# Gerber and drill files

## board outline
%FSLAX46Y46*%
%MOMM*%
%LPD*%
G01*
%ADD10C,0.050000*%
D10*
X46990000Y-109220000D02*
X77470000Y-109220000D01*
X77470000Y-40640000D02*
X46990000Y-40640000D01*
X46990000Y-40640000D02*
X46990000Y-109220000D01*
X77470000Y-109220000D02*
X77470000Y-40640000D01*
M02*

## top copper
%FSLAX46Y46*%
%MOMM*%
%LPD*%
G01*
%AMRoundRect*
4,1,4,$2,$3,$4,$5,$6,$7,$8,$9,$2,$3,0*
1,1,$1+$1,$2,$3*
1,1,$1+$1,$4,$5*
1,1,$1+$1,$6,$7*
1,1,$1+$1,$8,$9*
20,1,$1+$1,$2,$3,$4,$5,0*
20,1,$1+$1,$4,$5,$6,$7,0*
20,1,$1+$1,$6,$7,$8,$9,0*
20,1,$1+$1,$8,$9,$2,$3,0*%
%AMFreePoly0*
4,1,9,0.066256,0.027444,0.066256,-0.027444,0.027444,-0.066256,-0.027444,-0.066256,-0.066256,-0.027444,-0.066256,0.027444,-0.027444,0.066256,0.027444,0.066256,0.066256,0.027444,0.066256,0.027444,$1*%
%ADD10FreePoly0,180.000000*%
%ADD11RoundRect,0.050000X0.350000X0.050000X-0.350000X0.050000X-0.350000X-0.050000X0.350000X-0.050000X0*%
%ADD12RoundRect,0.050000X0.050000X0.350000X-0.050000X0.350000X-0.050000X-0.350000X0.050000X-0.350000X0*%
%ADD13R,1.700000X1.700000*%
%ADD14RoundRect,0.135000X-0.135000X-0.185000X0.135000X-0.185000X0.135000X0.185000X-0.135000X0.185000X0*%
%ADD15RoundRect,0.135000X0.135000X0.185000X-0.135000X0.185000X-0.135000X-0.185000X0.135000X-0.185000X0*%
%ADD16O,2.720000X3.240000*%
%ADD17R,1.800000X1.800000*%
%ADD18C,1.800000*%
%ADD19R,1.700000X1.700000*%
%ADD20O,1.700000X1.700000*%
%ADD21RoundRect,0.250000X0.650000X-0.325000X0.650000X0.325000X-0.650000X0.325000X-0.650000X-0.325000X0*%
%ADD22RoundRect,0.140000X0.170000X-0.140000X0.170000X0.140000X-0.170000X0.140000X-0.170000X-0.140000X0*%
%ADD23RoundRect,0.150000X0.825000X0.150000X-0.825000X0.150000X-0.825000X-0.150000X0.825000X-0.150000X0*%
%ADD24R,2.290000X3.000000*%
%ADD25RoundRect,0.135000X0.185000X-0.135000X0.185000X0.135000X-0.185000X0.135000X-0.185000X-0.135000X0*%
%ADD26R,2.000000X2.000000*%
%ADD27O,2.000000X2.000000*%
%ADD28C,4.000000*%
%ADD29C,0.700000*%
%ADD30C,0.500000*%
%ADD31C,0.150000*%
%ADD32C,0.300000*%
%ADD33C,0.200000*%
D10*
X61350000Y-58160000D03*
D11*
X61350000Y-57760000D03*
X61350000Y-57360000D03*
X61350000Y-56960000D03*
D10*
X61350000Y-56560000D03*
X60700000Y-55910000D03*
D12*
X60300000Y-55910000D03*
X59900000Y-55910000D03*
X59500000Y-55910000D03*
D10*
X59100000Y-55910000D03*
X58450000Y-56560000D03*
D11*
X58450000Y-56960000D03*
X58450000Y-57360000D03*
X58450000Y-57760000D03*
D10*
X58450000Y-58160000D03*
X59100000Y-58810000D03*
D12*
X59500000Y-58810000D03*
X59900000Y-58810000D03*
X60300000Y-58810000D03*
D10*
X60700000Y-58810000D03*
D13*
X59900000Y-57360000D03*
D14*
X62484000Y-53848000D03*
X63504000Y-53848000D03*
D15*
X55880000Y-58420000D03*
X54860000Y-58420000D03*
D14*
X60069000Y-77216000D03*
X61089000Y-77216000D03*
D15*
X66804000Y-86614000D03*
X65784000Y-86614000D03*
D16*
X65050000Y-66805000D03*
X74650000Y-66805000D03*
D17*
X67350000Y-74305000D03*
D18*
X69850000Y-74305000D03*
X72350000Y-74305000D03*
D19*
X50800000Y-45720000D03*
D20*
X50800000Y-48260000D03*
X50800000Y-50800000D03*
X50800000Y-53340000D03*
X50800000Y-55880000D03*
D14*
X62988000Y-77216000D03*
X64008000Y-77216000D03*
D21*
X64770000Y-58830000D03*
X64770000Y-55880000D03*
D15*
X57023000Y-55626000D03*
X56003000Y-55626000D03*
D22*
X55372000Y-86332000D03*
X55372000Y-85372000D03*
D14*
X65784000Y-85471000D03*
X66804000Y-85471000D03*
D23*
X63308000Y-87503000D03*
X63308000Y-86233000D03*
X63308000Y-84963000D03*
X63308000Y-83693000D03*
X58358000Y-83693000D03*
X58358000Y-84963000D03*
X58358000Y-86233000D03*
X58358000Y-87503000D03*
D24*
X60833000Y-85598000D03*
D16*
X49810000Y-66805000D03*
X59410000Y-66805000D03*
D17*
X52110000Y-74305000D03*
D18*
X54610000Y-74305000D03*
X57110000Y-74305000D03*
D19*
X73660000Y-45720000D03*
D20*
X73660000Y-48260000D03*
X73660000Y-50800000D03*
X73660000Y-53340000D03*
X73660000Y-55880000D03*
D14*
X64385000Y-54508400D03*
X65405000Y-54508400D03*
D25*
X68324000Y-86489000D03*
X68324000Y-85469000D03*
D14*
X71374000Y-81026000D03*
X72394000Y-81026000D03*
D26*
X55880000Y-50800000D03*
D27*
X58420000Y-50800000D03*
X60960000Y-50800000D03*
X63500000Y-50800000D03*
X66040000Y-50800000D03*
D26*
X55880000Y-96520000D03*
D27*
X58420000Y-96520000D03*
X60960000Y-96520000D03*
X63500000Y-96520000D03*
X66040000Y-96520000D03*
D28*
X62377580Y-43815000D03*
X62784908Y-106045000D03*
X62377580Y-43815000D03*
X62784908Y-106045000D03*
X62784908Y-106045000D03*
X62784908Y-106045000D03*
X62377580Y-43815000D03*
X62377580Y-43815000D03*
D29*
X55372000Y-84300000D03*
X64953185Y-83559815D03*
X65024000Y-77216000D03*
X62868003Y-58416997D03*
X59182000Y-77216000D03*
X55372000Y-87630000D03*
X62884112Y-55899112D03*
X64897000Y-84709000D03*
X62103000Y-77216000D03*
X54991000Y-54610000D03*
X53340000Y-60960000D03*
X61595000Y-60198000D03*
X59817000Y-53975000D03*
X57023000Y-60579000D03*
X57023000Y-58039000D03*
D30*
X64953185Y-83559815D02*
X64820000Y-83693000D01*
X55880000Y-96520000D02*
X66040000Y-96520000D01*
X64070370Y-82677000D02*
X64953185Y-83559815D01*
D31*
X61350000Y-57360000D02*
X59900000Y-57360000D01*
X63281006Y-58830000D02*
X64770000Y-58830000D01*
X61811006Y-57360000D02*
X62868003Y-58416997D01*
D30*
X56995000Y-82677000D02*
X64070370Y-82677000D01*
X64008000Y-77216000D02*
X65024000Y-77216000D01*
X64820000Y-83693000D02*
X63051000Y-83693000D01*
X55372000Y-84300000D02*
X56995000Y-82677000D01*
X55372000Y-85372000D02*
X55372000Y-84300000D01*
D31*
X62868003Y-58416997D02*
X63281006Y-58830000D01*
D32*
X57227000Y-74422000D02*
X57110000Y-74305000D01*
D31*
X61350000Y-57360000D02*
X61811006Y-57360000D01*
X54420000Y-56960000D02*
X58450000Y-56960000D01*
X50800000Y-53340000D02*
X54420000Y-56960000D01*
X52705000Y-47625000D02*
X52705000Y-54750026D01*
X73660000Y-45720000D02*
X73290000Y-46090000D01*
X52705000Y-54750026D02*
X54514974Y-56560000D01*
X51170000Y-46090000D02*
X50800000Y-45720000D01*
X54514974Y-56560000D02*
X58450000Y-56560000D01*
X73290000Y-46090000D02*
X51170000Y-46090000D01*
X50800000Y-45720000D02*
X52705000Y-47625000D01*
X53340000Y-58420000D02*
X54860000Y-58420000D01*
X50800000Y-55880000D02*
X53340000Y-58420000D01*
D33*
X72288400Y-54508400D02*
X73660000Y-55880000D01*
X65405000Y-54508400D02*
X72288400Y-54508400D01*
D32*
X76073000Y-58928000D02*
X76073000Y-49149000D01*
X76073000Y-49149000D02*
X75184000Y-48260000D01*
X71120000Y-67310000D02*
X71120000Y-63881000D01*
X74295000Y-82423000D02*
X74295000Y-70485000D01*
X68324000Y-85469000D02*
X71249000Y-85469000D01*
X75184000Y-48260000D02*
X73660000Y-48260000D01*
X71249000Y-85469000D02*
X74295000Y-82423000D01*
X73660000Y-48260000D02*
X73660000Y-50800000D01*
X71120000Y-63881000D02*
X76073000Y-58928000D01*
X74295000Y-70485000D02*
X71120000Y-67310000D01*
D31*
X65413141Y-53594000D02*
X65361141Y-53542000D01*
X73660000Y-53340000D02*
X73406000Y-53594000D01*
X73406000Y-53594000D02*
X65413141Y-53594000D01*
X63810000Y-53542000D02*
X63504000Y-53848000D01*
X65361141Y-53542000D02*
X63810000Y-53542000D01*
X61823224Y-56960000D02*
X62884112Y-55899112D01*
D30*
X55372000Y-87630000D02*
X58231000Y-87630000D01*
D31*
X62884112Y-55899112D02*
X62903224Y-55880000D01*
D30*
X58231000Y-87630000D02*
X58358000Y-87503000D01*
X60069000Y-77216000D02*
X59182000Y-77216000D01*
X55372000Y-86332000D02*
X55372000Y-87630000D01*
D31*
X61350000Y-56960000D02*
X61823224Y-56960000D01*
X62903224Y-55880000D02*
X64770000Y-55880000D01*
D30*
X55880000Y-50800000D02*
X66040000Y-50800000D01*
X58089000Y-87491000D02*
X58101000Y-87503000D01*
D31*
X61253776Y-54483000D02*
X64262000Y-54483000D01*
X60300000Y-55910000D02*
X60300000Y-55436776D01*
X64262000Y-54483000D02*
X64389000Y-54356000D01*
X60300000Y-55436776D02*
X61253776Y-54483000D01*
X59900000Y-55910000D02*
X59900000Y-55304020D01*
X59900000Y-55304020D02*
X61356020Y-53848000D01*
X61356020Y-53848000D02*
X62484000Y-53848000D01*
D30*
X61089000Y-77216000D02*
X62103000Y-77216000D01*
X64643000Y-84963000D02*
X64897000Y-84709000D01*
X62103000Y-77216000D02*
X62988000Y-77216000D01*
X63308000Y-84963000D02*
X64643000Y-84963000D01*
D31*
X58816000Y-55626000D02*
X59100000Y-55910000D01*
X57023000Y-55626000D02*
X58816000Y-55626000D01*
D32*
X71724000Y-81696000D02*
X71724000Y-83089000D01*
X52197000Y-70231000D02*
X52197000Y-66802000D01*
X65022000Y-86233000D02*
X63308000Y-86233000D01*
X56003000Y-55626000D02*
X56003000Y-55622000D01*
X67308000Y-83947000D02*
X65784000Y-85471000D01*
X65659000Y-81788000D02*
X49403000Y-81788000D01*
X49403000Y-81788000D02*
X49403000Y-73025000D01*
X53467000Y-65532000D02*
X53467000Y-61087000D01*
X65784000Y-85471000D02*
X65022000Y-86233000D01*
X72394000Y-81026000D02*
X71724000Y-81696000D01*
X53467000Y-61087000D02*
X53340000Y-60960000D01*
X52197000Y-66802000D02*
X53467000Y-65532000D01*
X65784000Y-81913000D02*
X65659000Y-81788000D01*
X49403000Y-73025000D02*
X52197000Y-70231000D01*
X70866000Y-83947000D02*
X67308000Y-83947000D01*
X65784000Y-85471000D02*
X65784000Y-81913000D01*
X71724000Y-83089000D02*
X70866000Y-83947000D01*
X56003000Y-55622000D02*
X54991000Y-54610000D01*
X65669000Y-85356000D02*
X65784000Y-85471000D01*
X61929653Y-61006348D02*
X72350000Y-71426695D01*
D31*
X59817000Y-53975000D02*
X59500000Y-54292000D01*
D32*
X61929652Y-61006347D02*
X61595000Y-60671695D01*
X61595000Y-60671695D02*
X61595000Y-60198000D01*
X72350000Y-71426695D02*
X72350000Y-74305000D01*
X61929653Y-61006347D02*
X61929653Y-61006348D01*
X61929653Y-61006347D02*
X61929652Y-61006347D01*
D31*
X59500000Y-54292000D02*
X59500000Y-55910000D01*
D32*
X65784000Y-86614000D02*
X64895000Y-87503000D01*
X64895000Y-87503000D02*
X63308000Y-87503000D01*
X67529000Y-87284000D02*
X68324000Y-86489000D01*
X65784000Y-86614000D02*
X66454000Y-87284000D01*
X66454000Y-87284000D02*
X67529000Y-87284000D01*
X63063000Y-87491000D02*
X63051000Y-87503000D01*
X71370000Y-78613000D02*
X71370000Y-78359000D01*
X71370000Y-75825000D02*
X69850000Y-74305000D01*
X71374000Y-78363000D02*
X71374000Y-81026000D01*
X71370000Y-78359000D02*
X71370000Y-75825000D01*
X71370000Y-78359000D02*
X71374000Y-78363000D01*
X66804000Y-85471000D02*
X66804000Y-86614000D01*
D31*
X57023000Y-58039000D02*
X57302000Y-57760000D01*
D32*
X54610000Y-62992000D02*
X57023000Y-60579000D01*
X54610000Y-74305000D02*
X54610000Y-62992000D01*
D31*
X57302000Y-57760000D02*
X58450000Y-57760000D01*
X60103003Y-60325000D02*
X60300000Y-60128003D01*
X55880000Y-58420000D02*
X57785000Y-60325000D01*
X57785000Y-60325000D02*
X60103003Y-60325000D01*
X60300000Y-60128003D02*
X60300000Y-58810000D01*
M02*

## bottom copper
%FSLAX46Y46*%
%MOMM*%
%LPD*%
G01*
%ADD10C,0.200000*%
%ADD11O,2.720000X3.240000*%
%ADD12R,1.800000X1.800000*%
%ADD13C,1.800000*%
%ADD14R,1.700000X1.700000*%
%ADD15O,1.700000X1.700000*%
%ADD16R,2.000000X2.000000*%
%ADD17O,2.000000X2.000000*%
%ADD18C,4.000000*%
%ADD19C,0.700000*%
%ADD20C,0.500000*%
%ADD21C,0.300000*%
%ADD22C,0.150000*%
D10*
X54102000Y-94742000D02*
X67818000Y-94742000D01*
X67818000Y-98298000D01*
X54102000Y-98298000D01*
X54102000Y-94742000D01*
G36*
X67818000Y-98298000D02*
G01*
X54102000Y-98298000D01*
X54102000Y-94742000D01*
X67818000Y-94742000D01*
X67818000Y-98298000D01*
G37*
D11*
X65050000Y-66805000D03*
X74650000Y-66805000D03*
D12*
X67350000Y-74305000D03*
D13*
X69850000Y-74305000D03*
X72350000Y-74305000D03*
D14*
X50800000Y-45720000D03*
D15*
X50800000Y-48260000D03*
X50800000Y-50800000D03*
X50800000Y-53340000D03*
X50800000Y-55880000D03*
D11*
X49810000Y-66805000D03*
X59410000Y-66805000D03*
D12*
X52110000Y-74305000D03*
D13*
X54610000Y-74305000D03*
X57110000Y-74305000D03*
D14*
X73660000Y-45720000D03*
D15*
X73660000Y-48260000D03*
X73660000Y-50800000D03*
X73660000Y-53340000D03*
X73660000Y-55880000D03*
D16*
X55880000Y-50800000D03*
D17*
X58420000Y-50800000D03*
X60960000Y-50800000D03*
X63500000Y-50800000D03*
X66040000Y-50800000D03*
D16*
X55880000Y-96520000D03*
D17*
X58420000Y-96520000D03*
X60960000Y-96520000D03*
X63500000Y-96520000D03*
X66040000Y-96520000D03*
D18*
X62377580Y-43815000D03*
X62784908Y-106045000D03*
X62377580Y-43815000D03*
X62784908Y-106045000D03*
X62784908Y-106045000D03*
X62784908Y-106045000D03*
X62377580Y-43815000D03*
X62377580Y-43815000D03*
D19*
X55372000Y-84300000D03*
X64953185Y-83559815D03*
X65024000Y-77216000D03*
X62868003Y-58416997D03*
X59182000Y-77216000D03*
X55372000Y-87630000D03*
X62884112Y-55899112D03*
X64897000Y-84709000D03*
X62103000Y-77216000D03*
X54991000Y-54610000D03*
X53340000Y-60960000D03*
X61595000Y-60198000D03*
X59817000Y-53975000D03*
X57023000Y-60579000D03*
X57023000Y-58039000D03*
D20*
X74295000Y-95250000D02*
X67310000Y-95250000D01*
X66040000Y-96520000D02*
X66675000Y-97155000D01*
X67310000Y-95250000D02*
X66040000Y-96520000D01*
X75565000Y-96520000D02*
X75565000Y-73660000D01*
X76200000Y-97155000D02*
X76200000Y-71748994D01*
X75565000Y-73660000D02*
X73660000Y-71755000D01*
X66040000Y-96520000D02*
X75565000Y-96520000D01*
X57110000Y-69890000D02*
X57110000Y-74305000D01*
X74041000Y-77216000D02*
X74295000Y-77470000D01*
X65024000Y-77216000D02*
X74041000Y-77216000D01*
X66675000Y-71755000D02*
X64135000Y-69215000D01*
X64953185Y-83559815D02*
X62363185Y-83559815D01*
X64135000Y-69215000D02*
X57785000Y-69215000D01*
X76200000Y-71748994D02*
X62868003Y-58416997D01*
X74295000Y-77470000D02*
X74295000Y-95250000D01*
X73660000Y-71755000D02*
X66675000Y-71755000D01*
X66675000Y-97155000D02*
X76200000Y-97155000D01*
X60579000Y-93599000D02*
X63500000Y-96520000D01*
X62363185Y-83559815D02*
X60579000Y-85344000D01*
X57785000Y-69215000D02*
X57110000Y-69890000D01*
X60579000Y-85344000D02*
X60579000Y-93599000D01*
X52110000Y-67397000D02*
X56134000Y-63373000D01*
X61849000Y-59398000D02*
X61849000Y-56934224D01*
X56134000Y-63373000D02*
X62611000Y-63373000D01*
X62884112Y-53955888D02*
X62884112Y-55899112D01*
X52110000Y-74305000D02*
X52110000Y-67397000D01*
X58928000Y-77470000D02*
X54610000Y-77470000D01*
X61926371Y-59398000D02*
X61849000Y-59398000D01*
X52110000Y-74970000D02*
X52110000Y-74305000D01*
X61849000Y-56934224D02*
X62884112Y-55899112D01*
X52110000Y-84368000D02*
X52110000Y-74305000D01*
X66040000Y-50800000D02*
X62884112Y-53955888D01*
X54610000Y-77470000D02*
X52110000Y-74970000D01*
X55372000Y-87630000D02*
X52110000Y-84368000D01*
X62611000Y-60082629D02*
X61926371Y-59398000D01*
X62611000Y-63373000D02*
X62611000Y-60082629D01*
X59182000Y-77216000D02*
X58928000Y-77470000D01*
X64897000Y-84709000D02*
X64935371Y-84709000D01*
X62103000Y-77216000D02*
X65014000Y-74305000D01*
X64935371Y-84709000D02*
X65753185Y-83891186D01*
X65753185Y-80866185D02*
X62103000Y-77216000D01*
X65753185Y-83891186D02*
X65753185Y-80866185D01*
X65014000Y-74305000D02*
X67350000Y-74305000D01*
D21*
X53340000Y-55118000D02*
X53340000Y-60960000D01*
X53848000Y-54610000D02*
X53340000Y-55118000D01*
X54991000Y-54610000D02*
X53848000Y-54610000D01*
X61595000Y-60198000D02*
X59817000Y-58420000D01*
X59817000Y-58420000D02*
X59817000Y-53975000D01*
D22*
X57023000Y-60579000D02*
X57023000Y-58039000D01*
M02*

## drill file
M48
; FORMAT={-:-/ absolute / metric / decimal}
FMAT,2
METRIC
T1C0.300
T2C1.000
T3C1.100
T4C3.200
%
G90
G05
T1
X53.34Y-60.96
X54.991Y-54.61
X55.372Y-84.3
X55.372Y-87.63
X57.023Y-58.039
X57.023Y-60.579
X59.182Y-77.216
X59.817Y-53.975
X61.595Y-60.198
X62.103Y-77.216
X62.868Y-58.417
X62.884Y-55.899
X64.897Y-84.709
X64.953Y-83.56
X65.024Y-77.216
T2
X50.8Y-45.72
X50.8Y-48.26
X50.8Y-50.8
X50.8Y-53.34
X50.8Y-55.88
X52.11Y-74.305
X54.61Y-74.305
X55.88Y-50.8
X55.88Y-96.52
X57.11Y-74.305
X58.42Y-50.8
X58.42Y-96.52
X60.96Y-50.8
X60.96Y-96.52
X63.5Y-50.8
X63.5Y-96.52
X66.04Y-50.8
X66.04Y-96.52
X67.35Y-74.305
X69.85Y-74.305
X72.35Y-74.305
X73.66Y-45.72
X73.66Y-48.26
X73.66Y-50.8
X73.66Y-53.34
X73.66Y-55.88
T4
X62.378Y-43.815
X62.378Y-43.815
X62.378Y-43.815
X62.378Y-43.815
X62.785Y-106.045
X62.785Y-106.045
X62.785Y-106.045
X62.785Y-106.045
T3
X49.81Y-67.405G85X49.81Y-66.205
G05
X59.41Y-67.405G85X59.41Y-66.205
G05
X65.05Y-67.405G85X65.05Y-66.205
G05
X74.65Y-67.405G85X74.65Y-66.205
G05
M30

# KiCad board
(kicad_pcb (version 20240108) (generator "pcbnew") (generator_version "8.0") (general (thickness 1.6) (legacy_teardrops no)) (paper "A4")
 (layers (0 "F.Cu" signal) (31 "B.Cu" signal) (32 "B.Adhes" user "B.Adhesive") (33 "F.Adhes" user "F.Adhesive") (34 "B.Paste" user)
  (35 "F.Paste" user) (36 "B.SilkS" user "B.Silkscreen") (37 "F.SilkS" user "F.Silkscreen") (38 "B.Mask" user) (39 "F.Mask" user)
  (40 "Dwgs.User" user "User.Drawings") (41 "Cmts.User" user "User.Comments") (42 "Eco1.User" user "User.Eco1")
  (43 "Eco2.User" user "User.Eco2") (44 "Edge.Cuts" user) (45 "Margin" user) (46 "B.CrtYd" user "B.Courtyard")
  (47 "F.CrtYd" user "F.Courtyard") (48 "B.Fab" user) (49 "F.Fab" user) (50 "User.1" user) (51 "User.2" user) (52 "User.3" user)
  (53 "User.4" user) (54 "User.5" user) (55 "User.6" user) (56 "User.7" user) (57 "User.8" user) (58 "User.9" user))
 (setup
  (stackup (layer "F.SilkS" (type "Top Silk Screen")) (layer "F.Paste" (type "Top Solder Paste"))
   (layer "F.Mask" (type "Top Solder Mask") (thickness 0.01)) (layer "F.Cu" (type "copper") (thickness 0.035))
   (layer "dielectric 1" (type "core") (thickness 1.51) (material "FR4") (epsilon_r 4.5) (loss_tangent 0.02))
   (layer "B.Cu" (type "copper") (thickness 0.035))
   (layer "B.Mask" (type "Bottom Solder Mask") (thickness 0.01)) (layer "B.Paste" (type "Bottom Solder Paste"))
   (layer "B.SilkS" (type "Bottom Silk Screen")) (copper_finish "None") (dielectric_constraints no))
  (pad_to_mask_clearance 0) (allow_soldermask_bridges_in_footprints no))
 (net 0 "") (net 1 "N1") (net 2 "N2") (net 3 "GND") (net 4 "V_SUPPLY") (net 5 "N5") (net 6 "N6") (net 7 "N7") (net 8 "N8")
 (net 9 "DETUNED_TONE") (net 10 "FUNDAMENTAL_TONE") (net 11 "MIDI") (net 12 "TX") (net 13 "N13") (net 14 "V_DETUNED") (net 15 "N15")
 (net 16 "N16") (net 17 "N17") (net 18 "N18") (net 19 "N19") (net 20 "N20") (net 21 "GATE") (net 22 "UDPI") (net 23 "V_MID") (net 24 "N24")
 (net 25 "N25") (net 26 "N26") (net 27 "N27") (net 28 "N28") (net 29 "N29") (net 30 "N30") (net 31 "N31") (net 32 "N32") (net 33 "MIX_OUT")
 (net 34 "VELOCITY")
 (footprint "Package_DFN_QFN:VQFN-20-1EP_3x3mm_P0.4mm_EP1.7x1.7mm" (layer "F.Cu") (at 59.9 57.36 180)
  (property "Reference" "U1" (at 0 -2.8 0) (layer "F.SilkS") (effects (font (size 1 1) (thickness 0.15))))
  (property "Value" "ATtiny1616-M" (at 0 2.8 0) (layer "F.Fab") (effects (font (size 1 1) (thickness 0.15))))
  (pad "" smd roundrect (at -0.425 -0.425 180) (size 0.69 0.69) (layers "F.Paste") (roundrect_rratio 0.25))
  (pad "" smd roundrect (at -0.425 0.425 180) (size 0.69 0.69) (layers "F.Paste") (roundrect_rratio 0.25))
  (pad "" smd roundrect (at 0.425 -0.425 180) (size 0.69 0.69) (layers "F.Paste") (roundrect_rratio 0.25))
  (pad "" smd roundrect (at 0.425 0.425 180) (size 0.69 0.69) (layers "F.Paste") (roundrect_rratio 0.25))
  (pad "1" smd custom (at -1.45 -0.8 180) (size 0.143431 0.143431) (layers "F.Cu" "F.Paste" "F.Mask") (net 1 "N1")
   (options (clearance outline) (anchor circle)) (primitives))
  (pad "2" smd roundrect (at -1.45 -0.4 180) (size 0.8 0.2) (layers "F.Cu" "F.Paste" "F.Mask") (roundrect_rratio 0.25) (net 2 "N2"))
  (pad "3" smd roundrect (at -1.45 0 180) (size 0.8 0.2) (layers "F.Cu" "F.Paste" "F.Mask") (roundrect_rratio 0.25) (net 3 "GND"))
  (pad "4" smd roundrect (at -1.45 0.4 180) (size 0.8 0.2) (layers "F.Cu" "F.Paste" "F.Mask") (roundrect_rratio 0.25) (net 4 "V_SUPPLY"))
  (pad "5" smd custom (at -1.45 0.8 180) (size 0.143431 0.143431) (layers "F.Cu" "F.Paste" "F.Mask") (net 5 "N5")
   (options (clearance outline) (anchor circle)) (primitives))
  (pad "6" smd custom (at -0.8 1.45 180) (size 0.143431 0.143431) (layers "F.Cu" "F.Paste" "F.Mask") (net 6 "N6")
   (options (clearance outline) (anchor circle)) (primitives))
  (pad "7" smd roundrect (at -0.4 1.45 180) (size 0.2 0.8) (layers "F.Cu" "F.Paste" "F.Mask") (roundrect_rratio 0.25) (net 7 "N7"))
  (pad "8" smd roundrect (at 0 1.45 180) (size 0.2 0.8) (layers "F.Cu" "F.Paste" "F.Mask") (roundrect_rratio 0.25) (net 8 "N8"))
  (pad "9" smd roundrect (at 0.4 1.45 180) (size 0.2 0.8) (layers "F.Cu" "F.Paste" "F.Mask") (roundrect_rratio 0.25) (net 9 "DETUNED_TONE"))
  (pad "10" smd custom (at 0.8 1.45 180) (size 0.143431 0.143431) (layers "F.Cu" "F.Paste" "F.Mask") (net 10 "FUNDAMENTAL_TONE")
   (options (clearance outline) (anchor circle)) (primitives))
  (pad "11" smd custom (at 1.45 0.8 180) (size 0.143431 0.143431) (layers "F.Cu" "F.Paste" "F.Mask") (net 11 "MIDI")
   (options (clearance outline) (anchor circle)) (primitives))
  (pad "12" smd roundrect (at 1.45 0.4 180) (size 0.8 0.2) (layers "F.Cu" "F.Paste" "F.Mask") (roundrect_rratio 0.25) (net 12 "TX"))
  (pad "13" smd roundrect (at 1.45 0 180) (size 0.8 0.2) (layers "F.Cu" "F.Paste" "F.Mask") (roundrect_rratio 0.25) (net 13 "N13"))
  (pad "14" smd roundrect (at 1.45 -0.4 180) (size 0.8 0.2) (layers "F.Cu" "F.Paste" "F.Mask") (roundrect_rratio 0.25) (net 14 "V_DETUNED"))
  (pad "15" smd custom (at 1.45 -0.8 180) (size 0.143431 0.143431) (layers "F.Cu" "F.Paste" "F.Mask") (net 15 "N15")
   (options (clearance outline) (anchor circle)) (primitives))
  (pad "16" smd custom (at 0.8 -1.45 180) (size 0.143431 0.143431) (layers "F.Cu" "F.Paste" "F.Mask") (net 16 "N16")
   (options (clearance outline) (anchor circle)) (primitives))
  (pad "17" smd roundrect (at 0.4 -1.45 180) (size 0.2 0.8) (layers "F.Cu" "F.Paste" "F.Mask") (roundrect_rratio 0.25) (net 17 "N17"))
  (pad "18" smd roundrect (at 0 -1.45 180) (size 0.2 0.8) (layers "F.Cu" "F.Paste" "F.Mask") (roundrect_rratio 0.25) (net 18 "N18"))
  (pad "19" smd roundrect (at -0.4 -1.45 180) (size 0.2 0.8) (layers "F.Cu" "F.Paste" "F.Mask") (roundrect_rratio 0.25) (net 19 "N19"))
  (pad "20" smd custom (at -0.8 -1.45 180) (size 0.143431 0.143431) (layers "F.Cu" "F.Paste" "F.Mask") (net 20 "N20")
   (options (clearance outline) (anchor circle)) (primitives))
  (pad "21" smd rect (at 0 0 180) (size 1.7 1.7) (layers "F.Cu" "F.Mask") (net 3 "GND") (zone_connect 2)))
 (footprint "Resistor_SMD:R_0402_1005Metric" (layer "F.Cu") (at 62.994 53.848)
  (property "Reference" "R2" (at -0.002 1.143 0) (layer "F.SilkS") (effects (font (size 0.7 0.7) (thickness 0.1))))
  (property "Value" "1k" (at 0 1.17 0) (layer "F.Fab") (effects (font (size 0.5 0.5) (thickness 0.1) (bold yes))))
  (pad "1" smd roundrect (at -0.51 0) (size 0.54 0.64) (layers "F.Cu" "F.Paste" "F.Mask") (roundrect_rratio 0.25) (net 8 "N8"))
  (pad "2" smd roundrect (at 0.51 0) (size 0.54 0.64) (layers "F.Cu" "F.Paste" "F.Mask") (roundrect_rratio 0.25) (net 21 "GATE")))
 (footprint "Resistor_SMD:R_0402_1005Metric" (layer "F.Cu") (at 55.37 58.42 180)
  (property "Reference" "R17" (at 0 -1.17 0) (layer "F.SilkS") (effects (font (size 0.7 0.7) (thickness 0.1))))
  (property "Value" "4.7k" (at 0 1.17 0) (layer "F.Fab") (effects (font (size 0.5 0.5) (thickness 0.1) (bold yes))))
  (pad "1" smd roundrect (at -0.51 0 180) (size 0.54 0.64) (layers "F.Cu" "F.Paste" "F.Mask") (roundrect_rratio 0.25) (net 19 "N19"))
  (pad "2" smd roundrect (at 0.51 0 180) (size 0.54 0.64) (layers "F.Cu" "F.Paste" "F.Mask") (roundrect_rratio 0.25) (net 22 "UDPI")))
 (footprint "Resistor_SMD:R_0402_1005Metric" (layer "F.Cu") (at 60.579 77.216)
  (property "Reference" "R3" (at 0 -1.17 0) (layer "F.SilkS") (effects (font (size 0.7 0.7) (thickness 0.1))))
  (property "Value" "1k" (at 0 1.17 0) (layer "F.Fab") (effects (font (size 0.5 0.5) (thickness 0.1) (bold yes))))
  (pad "1" smd roundrect (at -0.51 0) (size 0.54 0.64) (layers "F.Cu" "F.Paste" "F.Mask") (roundrect_rratio 0.25) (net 4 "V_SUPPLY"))
  (pad "2" smd roundrect (at 0.51 0) (size 0.54 0.64) (layers "F.Cu" "F.Paste" "F.Mask") (roundrect_rratio 0.25) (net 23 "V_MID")))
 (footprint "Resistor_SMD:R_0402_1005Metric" (layer "F.Cu") (at 66.294 86.614 180)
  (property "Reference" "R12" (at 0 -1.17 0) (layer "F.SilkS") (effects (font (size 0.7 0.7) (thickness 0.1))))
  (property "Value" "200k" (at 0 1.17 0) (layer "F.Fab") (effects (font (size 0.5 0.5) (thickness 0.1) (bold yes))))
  (pad "1" smd roundrect (at -0.51 0 180) (size 0.54 0.64) (layers "F.Cu" "F.Paste" "F.Mask") (roundrect_rratio 0.25) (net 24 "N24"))
  (pad "2" smd roundrect (at 0.51 0 180) (size 0.54 0.64) (layers "F.Cu" "F.Paste" "F.Mask") (roundrect_rratio 0.25) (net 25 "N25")))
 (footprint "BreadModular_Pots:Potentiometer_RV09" (layer "F.Cu") (at 67.35 74.305 90)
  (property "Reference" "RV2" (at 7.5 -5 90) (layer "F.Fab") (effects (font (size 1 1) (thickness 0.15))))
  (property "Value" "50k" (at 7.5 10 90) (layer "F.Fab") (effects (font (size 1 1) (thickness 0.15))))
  (pad "" thru_hole oval (at 7.5 -2.3 180) (size 2.72 3.24) (drill oval 1.1 2.3) (layers "*.Cu" "*.Mask") (remove_unused_layers no))
  (pad "" thru_hole oval (at 7.5 7.3 180) (size 2.72 3.24) (drill oval 1.1 2.3) (layers "*.Cu" "*.Mask") (remove_unused_layers no))
  (pad "1" thru_hole rect (at 0 0 180) (size 1.8 1.8) (drill 1) (layers "*.Cu" "*.Mask") (remove_unused_layers no) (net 23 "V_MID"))
  (pad "2" thru_hole circle (at 0 2.5 180) (size 1.8 1.8) (drill 1) (layers "*.Cu" "*.Mask") (remove_unused_layers no) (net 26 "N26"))
  (pad "3" thru_hole circle (at 0 5 180) (size 1.8 1.8) (drill 1) (layers "*.Cu" "*.Mask") (remove_unused_layers no) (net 9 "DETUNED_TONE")))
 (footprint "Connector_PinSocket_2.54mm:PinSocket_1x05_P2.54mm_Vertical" (layer "F.Cu") (at 50.8 45.72)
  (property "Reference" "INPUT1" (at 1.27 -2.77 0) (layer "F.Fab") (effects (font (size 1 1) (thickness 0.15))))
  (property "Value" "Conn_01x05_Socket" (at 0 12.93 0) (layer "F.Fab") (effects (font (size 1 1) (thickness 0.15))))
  (pad "1" thru_hole rect (at 0 0) (size 1.7 1.7) (drill 1) (layers "*.Cu" "*.Mask") (remove_unused_layers no) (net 11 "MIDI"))
  (pad "2" thru_hole oval (at 0 2.54) (size 1.7 1.7) (drill 1) (layers "*.Cu" "*.Mask") (remove_unused_layers no) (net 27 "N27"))
  (pad "3" thru_hole oval (at 0 5.08) (size 1.7 1.7) (drill 1) (layers "*.Cu" "*.Mask") (remove_unused_layers no) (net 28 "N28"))
  (pad "4" thru_hole oval (at 0 7.62) (size 1.7 1.7) (drill 1) (layers "*.Cu" "*.Mask") (remove_unused_layers no) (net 12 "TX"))
  (pad "5" thru_hole oval (at 0 10.16) (size 1.7 1.7) (drill 1) (layers "*.Cu" "*.Mask") (remove_unused_layers no) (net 22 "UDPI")))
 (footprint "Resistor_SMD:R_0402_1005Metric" (layer "F.Cu") (at 63.498 77.216)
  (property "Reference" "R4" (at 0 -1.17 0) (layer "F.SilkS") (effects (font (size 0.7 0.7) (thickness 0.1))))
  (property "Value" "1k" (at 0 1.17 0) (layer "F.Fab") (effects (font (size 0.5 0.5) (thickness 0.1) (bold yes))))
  (pad "1" smd roundrect (at -0.51 0) (size 0.54 0.64) (layers "F.Cu" "F.Paste" "F.Mask") (roundrect_rratio 0.25) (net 23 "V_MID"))
  (pad "2" smd roundrect (at 0.51 0) (size 0.54 0.64) (layers "F.Cu" "F.Paste" "F.Mask") (roundrect_rratio 0.25) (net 3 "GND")))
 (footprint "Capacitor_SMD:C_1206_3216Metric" (layer "F.Cu") (at 64.77 57.355 90)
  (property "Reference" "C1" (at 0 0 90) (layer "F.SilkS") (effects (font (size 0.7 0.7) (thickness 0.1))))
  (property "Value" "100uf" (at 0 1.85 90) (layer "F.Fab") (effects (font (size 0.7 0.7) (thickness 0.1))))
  (pad "1" smd roundrect (at -1.475 0 90) (size 1.15 1.8) (layers "F.Cu" "F.Paste" "F.Mask") (roundrect_rratio 0.217391) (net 3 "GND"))
  (pad "2" smd roundrect (at 1.475 0 90) (size 1.15 1.8) (layers "F.Cu" "F.Paste" "F.Mask") (roundrect_rratio 0.217391) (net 4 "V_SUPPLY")))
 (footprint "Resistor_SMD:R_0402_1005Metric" (layer "F.Cu") (at 56.513 55.626 180)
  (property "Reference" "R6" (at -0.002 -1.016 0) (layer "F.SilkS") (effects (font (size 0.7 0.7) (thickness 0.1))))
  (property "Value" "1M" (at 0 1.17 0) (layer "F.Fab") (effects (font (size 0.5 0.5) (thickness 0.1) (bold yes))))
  (pad "1" smd roundrect (at -0.51 0 180) (size 0.54 0.64) (layers "F.Cu" "F.Paste" "F.Mask") (roundrect_rratio 0.25)
   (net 10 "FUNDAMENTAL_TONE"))
  (pad "2" smd roundrect (at 0.51 0 180) (size 0.54 0.64) (layers "F.Cu" "F.Paste" "F.Mask") (roundrect_rratio 0.25) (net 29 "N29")))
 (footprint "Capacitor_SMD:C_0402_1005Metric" (layer "F.Cu") (at 55.372 85.852 90)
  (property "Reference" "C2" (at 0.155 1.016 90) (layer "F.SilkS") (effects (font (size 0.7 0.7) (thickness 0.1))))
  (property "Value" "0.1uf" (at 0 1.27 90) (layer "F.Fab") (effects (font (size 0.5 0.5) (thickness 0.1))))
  (pad "1" smd roundrect (at -0.48 0 90) (size 0.56 0.62) (layers "F.Cu" "F.Paste" "F.Mask") (roundrect_rratio 0.25) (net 4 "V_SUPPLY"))
  (pad "2" smd roundrect (at 0.48 0 90) (size 0.56 0.62) (layers "F.Cu" "F.Paste" "F.Mask") (roundrect_rratio 0.25) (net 3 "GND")))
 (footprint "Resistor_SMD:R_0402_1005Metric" (layer "F.Cu") (at 66.294 85.471)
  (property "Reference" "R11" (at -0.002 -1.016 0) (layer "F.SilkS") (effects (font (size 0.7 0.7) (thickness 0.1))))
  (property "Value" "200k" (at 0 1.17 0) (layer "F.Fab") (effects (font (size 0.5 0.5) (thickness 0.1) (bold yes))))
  (pad "1" smd roundrect (at -0.51 0) (size 0.54 0.64) (layers "F.Cu" "F.Paste" "F.Mask") (roundrect_rratio 0.25) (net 29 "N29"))
  (pad "2" smd roundrect (at 0.51 0) (size 0.54 0.64) (layers "F.Cu" "F.Paste" "F.Mask") (roundrect_rratio 0.25) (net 24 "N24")))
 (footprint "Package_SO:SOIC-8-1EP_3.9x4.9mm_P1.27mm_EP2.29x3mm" (layer "F.Cu") (at 60.833 85.598 180)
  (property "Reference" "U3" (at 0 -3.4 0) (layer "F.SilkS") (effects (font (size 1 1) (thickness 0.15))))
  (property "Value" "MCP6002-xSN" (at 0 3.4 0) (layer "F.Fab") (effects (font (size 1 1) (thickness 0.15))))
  (pad "" smd roundrect (at -0.57 -0.75 180) (size 0.92 1.21) (layers "F.Paste") (roundrect_rratio 0.25))
  (pad "" smd roundrect (at -0.57 0.75 180) (size 0.92 1.21) (layers "F.Paste") (roundrect_rratio 0.25))
  (pad "" smd roundrect (at 0.57 -0.75 180) (size 0.92 1.21) (layers "F.Paste") (roundrect_rratio 0.25))
  (pad "" smd roundrect (at 0.57 0.75 180) (size 0.92 1.21) (layers "F.Paste") (roundrect_rratio 0.25))
  (pad "1" smd roundrect (at -2.475 -1.905 180) (size 1.95 0.6) (layers "F.Cu" "F.Paste" "F.Mask") (roundrect_rratio 0.25) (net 25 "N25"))
  (pad "2" smd roundrect (at -2.475 -0.635 180) (size 1.95 0.6) (layers "F.Cu" "F.Paste" "F.Mask") (roundrect_rratio 0.25) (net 29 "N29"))
  (pad "3" smd roundrect (at -2.475 0.635 180) (size 1.95 0.6) (layers "F.Cu" "F.Paste" "F.Mask") (roundrect_rratio 0.25) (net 23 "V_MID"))
  (pad "4" smd roundrect (at -2.475 1.905 180) (size 1.95 0.6) (layers "F.Cu" "F.Paste" "F.Mask") (roundrect_rratio 0.25) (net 3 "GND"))
  (pad "5" smd roundrect (at 2.475 1.905 180) (size 1.95 0.6) (layers "F.Cu" "F.Paste" "F.Mask") (roundrect_rratio 0.25) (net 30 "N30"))
  (pad "6" smd roundrect (at 2.475 0.635 180) (size 1.95 0.6) (layers "F.Cu" "F.Paste" "F.Mask") (roundrect_rratio 0.25) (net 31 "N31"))
  (pad "7" smd roundrect (at 2.475 -0.635 180) (size 1.95 0.6) (layers "F.Cu" "F.Paste" "F.Mask") (roundrect_rratio 0.25) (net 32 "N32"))
  (pad "8" smd roundrect (at 2.475 -1.905 180) (size 1.95 0.6) (layers "F.Cu" "F.Paste" "F.Mask") (roundrect_rratio 0.25) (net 4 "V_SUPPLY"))
  (pad "9" smd rect (at 0 0 180) (size 2.29 3) (layers "F.Cu" "F.Mask") (zone_connect 2)))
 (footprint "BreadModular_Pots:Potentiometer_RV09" (layer "F.Cu") (at 52.11 74.305 90)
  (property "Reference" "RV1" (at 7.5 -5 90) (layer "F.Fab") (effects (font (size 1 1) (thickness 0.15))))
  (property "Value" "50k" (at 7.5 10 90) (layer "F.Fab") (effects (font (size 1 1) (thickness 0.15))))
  (pad "" thru_hole oval (at 7.5 -2.3 180) (size 2.72 3.24) (drill oval 1.1 2.3) (layers "*.Cu" "*.Mask") (remove_unused_layers no))
  (pad "" thru_hole oval (at 7.5 7.3 180) (size 2.72 3.24) (drill oval 1.1 2.3) (layers "*.Cu" "*.Mask") (remove_unused_layers no))
  (pad "1" thru_hole rect (at 0 0 180) (size 1.8 1.8) (drill 1) (layers "*.Cu" "*.Mask") (remove_unused_layers no) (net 4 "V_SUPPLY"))
  (pad "2" thru_hole circle (at 0 2.5 180) (size 1.8 1.8) (drill 1) (layers "*.Cu" "*.Mask") (remove_unused_layers no) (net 14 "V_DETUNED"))
  (pad "3" thru_hole circle (at 0 5 180) (size 1.8 1.8) (drill 1) (layers "*.Cu" "*.Mask") (remove_unused_layers no) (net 3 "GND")))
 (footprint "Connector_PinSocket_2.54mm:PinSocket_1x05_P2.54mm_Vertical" (layer "F.Cu") (at 73.66 45.72)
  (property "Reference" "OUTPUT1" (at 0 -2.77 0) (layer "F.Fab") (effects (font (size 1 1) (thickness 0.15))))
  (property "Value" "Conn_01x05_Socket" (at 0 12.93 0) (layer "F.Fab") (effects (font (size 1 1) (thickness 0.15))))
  (pad "1" thru_hole rect (at 0 0) (size 1.7 1.7) (drill 1) (layers "*.Cu" "*.Mask") (remove_unused_layers no) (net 11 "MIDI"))
  (pad "2" thru_hole oval (at 0 2.54) (size 1.7 1.7) (drill 1) (layers "*.Cu" "*.Mask") (remove_unused_layers no) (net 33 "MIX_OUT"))
  (pad "3" thru_hole oval (at 0 5.08) (size 1.7 1.7) (drill 1) (layers "*.Cu" "*.Mask") (remove_unused_layers no) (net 33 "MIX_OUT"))
  (pad "4" thru_hole oval (at 0 7.62) (size 1.7 1.7) (drill 1) (layers "*.Cu" "*.Mask") (remove_unused_layers no) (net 21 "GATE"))
  (pad "5" thru_hole oval (at 0 10.16) (size 1.7 1.7) (drill 1) (layers "*.Cu" "*.Mask") (remove_unused_layers no) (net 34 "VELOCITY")))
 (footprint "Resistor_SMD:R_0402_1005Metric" (layer "F.Cu") (at 64.895 54.5084)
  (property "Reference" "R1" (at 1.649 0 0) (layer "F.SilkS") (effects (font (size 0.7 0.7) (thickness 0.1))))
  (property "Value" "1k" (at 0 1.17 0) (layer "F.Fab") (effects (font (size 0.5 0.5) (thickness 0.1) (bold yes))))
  (pad "1" smd roundrect (at -0.51 0) (size 0.54 0.64) (layers "F.Cu" "F.Paste" "F.Mask") (roundrect_rratio 0.25) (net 7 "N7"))
  (pad "2" smd roundrect (at 0.51 0) (size 0.54 0.64) (layers "F.Cu" "F.Paste" "F.Mask") (roundrect_rratio 0.25) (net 34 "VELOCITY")))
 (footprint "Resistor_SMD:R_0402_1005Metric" (layer "F.Cu") (at 68.324 85.979 90)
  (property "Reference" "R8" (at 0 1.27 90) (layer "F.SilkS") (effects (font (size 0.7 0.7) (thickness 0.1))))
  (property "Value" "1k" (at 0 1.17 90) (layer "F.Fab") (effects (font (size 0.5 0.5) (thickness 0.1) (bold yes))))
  (pad "1" smd roundrect (at -0.51 0 90) (size 0.54 0.64) (layers "F.Cu" "F.Paste" "F.Mask") (roundrect_rratio 0.25) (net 25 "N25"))
  (pad "2" smd roundrect (at 0.51 0 90) (size 0.54 0.64) (layers "F.Cu" "F.Paste" "F.Mask") (roundrect_rratio 0.25) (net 33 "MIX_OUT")))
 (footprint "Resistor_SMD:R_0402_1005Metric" (layer "F.Cu") (at 71.884 81.026)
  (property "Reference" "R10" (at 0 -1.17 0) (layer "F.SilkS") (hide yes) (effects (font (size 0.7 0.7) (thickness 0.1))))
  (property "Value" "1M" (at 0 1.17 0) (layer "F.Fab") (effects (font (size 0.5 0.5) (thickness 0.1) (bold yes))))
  (pad "1" smd roundrect (at -0.51 0) (size 0.54 0.64) (layers "F.Cu" "F.Paste" "F.Mask") (roundrect_rratio 0.25) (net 26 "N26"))
  (pad "2" smd roundrect (at 0.51 0) (size 0.54 0.64) (layers "F.Cu" "F.Paste" "F.Mask") (roundrect_rratio 0.25) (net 29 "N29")))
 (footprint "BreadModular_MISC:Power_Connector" (layer "B.Cu") (at 55.88 50.8 -90)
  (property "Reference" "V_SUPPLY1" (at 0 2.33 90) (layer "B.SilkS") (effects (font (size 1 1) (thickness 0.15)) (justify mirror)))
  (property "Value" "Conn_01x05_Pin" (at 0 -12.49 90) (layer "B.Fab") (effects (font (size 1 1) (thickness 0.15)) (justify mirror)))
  (pad "1" thru_hole rect (at 0 0 270) (size 2 2) (drill 1) (layers "*.Cu" "*.Mask") (remove_unused_layers no) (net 4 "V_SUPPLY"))
  (pad "2" thru_hole oval (at 0 -2.54 270) (size 2 2) (drill 1) (layers "*.Cu" "*.Mask") (remove_unused_layers no) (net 4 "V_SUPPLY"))
  (pad "3" thru_hole oval (at 0 -5.08 270) (size 2 2) (drill 1) (layers "*.Cu" "*.Mask") (remove_unused_layers no) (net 4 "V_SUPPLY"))
  (pad "4" thru_hole oval (at 0 -7.62 270) (size 2 2) (drill 1) (layers "*.Cu" "*.Mask") (remove_unused_layers no) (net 4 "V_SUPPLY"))
  (pad "5" thru_hole oval (at 0 -10.16 270) (size 2 2) (drill 1) (layers "*.Cu" "*.Mask") (remove_unused_layers no) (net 4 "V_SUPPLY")))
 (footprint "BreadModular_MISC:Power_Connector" (layer "B.Cu") (at 55.88 96.52 -90)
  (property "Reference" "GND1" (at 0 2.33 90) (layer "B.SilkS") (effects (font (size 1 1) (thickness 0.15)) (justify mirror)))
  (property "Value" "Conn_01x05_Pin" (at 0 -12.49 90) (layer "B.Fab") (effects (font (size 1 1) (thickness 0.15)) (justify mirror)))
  (pad "1" thru_hole rect (at 0 0 270) (size 2 2) (drill 1) (layers "*.Cu" "*.Mask") (remove_unused_layers no) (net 3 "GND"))
  (pad "2" thru_hole oval (at 0 -2.54 270) (size 2 2) (drill 1) (layers "*.Cu" "*.Mask") (remove_unused_layers no) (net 3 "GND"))
  (pad "3" thru_hole oval (at 0 -5.08 270) (size 2 2) (drill 1) (layers "*.Cu" "*.Mask") (remove_unused_layers no) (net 3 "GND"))
  (pad "4" thru_hole oval (at 0 -7.62 270) (size 2 2) (drill 1) (layers "*.Cu" "*.Mask") (remove_unused_layers no) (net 3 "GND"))
  (pad "5" thru_hole oval (at 0 -10.16 270) (size 2 2) (drill 1) (layers "*.Cu" "*.Mask") (remove_unused_layers no) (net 3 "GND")))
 (gr_poly
  (pts (xy 54.102 94.742) (xy 67.818 94.742) (xy 67.818 98.298) (xy 54.102 98.298)) (stroke (width 0.2) (type solid)) (fill solid)
  (layer "B.Cu") (net 3))
 (gr_line (start 46.99 109.22) (end 77.47 109.22) (stroke (width 0.05) (type default)) (layer "Edge.Cuts"))
 (gr_line (start 77.47 40.64) (end 46.99 40.64) (stroke (width 0.05) (type default)) (layer "Edge.Cuts"))
 (gr_line (start 46.99 40.64) (end 46.99 109.22) (stroke (width 0.05) (type default)) (layer "Edge.Cuts"))
 (gr_line (start 77.47 109.22) (end 77.47 40.64) (stroke (width 0.05) (type default)) (layer "Edge.Cuts"))
 (via (at 62.37758 43.815) (size 4) (drill 3.2) (layers "F.Cu" "B.Cu") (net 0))
 (via (at 62.784908 106.045) (size 4) (drill 3.2) (layers "F.Cu" "B.Cu") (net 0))
 (via (at 62.37758 43.815) (size 4) (drill 3.2) (layers "F.Cu" "B.Cu") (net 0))
 (via (at 62.784908 106.045) (size 4) (drill 3.2) (layers "F.Cu" "B.Cu") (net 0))
 (via (at 62.784908 106.045) (size 4) (drill 3.2) (layers "F.Cu" "B.Cu") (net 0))
 (via (at 62.784908 106.045) (size 4) (drill 3.2) (layers "F.Cu" "B.Cu") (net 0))
 (via (at 62.37758 43.815) (size 4) (drill 3.2) (layers "F.Cu" "B.Cu") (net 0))
 (via (at 62.37758 43.815) (size 4) (drill 3.2) (layers "F.Cu" "B.Cu") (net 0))
 (segment (start 64.953185 83.559815) (end 64.82 83.693) (width 0.5) (layer "F.Cu") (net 3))
 (segment (start 55.88 96.52) (end 66.04 96.52) (width 0.5) (layer "F.Cu") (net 3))
 (segment (start 64.07037 82.677) (end 64.953185 83.559815) (width 0.5) (layer "F.Cu") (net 3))
 (segment (start 61.35 57.36) (end 59.9 57.36) (width 0.15) (layer "F.Cu") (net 3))
 (segment (start 63.281006 58.83) (end 64.77 58.83) (width 0.15) (layer "F.Cu") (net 3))
 (segment (start 61.811006 57.36) (end 62.868003 58.416997) (width 0.15) (layer "F.Cu") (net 3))
 (segment (start 56.995 82.677) (end 64.07037 82.677) (width 0.5) (layer "F.Cu") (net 3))
 (segment (start 64.008 77.216) (end 65.024 77.216) (width 0.5) (layer "F.Cu") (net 3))
 (segment (start 64.82 83.693) (end 63.051 83.693) (width 0.5) (layer "F.Cu") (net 3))
 (segment (start 55.372 84.3) (end 56.995 82.677) (width 0.5) (layer "F.Cu") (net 3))
 (segment (start 55.372 85.372) (end 55.372 84.3) (width 0.5) (layer "F.Cu") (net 3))
 (segment (start 62.868003 58.416997) (end 63.281006 58.83) (width 0.15) (layer "F.Cu") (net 3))
 (segment (start 57.227 74.422) (end 57.11 74.305) (width 0.3) (layer "F.Cu") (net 3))
 (segment (start 61.35 57.36) (end 61.811006 57.36) (width 0.15) (layer "F.Cu") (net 3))
 (via (at 55.372 84.3) (size 0.7) (drill 0.3) (layers "F.Cu" "B.Cu") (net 3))
 (via (at 64.953185 83.559815) (size 0.7) (drill 0.3) (layers "F.Cu" "B.Cu") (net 3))
 (via (at 65.024 77.216) (size 0.7) (drill 0.3) (layers "F.Cu" "B.Cu") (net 3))
 (via (at 62.868003 58.416997) (size 0.7) (drill 0.3) (layers "F.Cu" "B.Cu") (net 3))
 (segment (start 74.295 95.25) (end 67.31 95.25) (width 0.5) (layer "B.Cu") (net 3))
 (segment (start 66.04 96.52) (end 66.675 97.155) (width 0.5) (layer "B.Cu") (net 3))
 (segment (start 67.31 95.25) (end 66.04 96.52) (width 0.5) (layer "B.Cu") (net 3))
 (segment (start 75.565 96.52) (end 75.565 73.66) (width 0.5) (layer "B.Cu") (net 3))
 (segment (start 76.2 97.155) (end 76.2 71.748994) (width 0.5) (layer "B.Cu") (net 3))
 (segment (start 75.565 73.66) (end 73.66 71.755) (width 0.5) (layer "B.Cu") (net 3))
 (segment (start 66.04 96.52) (end 75.565 96.52) (width 0.5) (layer "B.Cu") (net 3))
 (segment (start 57.11 69.89) (end 57.11 74.305) (width 0.5) (layer "B.Cu") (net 3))
 (segment (start 74.041 77.216) (end 74.295 77.47) (width 0.5) (layer "B.Cu") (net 3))
 (segment (start 65.024 77.216) (end 74.041 77.216) (width 0.5) (layer "B.Cu") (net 3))
 (segment (start 66.675 71.755) (end 64.135 69.215) (width 0.5) (layer "B.Cu") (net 3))
 (segment (start 64.953185 83.559815) (end 62.363185 83.559815) (width 0.5) (layer "B.Cu") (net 3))
 (segment (start 64.135 69.215) (end 57.785 69.215) (width 0.5) (layer "B.Cu") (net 3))
 (segment (start 76.2 71.748994) (end 62.868003 58.416997) (width 0.5) (layer "B.Cu") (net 3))
 (segment (start 74.295 77.47) (end 74.295 95.25) (width 0.5) (layer "B.Cu") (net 3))
 (segment (start 73.66 71.755) (end 66.675 71.755) (width 0.5) (layer "B.Cu") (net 3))
 (segment (start 66.675 97.155) (end 76.2 97.155) (width 0.5) (layer "B.Cu") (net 3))
 (segment (start 60.579 93.599) (end 63.5 96.52) (width 0.5) (layer "B.Cu") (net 3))
 (segment (start 62.363185 83.559815) (end 60.579 85.344) (width 0.5) (layer "B.Cu") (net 3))
 (segment (start 57.785 69.215) (end 57.11 69.89) (width 0.5) (layer "B.Cu") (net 3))
 (segment (start 60.579 85.344) (end 60.579 93.599) (width 0.5) (layer "B.Cu") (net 3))
 (segment (start 54.42 56.96) (end 58.45 56.96) (width 0.15) (layer "F.Cu") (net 12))
 (segment (start 50.8 53.34) (end 54.42 56.96) (width 0.15) (layer "F.Cu") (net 12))
 (segment (start 52.705 47.625) (end 52.705 54.750026) (width 0.15) (layer "F.Cu") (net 11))
 (segment (start 73.66 45.72) (end 73.29 46.09) (width 0.15) (layer "F.Cu") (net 11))
 (segment (start 52.705 54.750026) (end 54.514974 56.56) (width 0.15) (layer "F.Cu") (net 11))
 (segment (start 51.17 46.09) (end 50.8 45.72) (width 0.15) (layer "F.Cu") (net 11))
 (segment (start 54.514974 56.56) (end 58.45 56.56) (width 0.15) (layer "F.Cu") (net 11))
 (segment (start 73.29 46.09) (end 51.17 46.09) (width 0.15) (layer "F.Cu") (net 11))
 (segment (start 50.8 45.72) (end 52.705 47.625) (width 0.15) (layer "F.Cu") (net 11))
 (segment (start 53.34 58.42) (end 54.86 58.42) (width 0.15) (layer "F.Cu") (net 22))
 (segment (start 50.8 55.88) (end 53.34 58.42) (width 0.15) (layer "F.Cu") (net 22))
 (segment (start 72.2884 54.5084) (end 73.66 55.88) (width 0.2) (layer "F.Cu") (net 34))
 (segment (start 65.405 54.5084) (end 72.2884 54.5084) (width 0.2) (layer "F.Cu") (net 34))
 (segment (start 76.073 58.928) (end 76.073 49.149) (width 0.3) (layer "F.Cu") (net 33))
 (segment (start 76.073 49.149) (end 75.184 48.26) (width 0.3) (layer "F.Cu") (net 33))
 (segment (start 71.12 67.31) (end 71.12 63.881) (width 0.3) (layer "F.Cu") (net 33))
 (segment (start 74.295 82.423) (end 74.295 70.485) (width 0.3) (layer "F.Cu") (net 33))
 (segment (start 68.324 85.469) (end 71.249 85.469) (width 0.3) (layer "F.Cu") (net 33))
 (segment (start 75.184 48.26) (end 73.66 48.26) (width 0.3) (layer "F.Cu") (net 33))
 (segment (start 71.249 85.469) (end 74.295 82.423) (width 0.3) (layer "F.Cu") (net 33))
 (segment (start 73.66 48.26) (end 73.66 50.8) (width 0.3) (layer "F.Cu") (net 33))
 (segment (start 71.12 63.881) (end 76.073 58.928) (width 0.3) (layer "F.Cu") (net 33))
 (segment (start 74.295 70.485) (end 71.12 67.31) (width 0.3) (layer "F.Cu") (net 33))
 (segment (start 65.413141 53.594) (end 65.361141 53.542) (width 0.15) (layer "F.Cu") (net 21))
 (segment (start 73.66 53.34) (end 73.406 53.594) (width 0.15) (layer "F.Cu") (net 21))
 (segment (start 73.406 53.594) (end 65.413141 53.594) (width 0.15) (layer "F.Cu") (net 21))
 (segment (start 63.81 53.542) (end 63.504 53.848) (width 0.15) (layer "F.Cu") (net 21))
 (segment (start 65.361141 53.542) (end 63.81 53.542) (width 0.15) (layer "F.Cu") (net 21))
 (segment (start 61.823224 56.96) (end 62.884112 55.899112) (width 0.15) (layer "F.Cu") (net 4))
 (segment (start 55.372 87.63) (end 58.231 87.63) (width 0.5) (layer "F.Cu") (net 4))
 (segment (start 62.884112 55.899112) (end 62.903224 55.88) (width 0.15) (layer "F.Cu") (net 4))
 (segment (start 58.231 87.63) (end 58.358 87.503) (width 0.5) (layer "F.Cu") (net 4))
 (segment (start 60.069 77.216) (end 59.182 77.216) (width 0.5) (layer "F.Cu") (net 4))
 (segment (start 55.372 86.332) (end 55.372 87.63) (width 0.5) (layer "F.Cu") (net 4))
 (segment (start 61.35 56.96) (end 61.823224 56.96) (width 0.15) (layer "F.Cu") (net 4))
 (segment (start 62.903224 55.88) (end 64.77 55.88) (width 0.15) (layer "F.Cu") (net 4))
 (segment (start 55.88 50.8) (end 66.04 50.8) (width 0.5) (layer "F.Cu") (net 4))
 (segment (start 58.089 87.491) (end 58.101 87.503) (width 0.5) (layer "F.Cu") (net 4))
 (via (at 59.182 77.216) (size 0.7) (drill 0.3) (layers "F.Cu" "B.Cu") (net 4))
 (via (at 55.372 87.63) (size 0.7) (drill 0.3) (layers "F.Cu" "B.Cu") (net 4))
 (via (at 62.884112 55.899112) (size 0.7) (drill 0.3) (layers "F.Cu" "B.Cu") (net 4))
 (segment (start 52.11 67.397) (end 56.134 63.373) (width 0.5) (layer "B.Cu") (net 4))
 (segment (start 61.849 59.398) (end 61.849 56.934224) (width 0.5) (layer "B.Cu") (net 4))
 (segment (start 56.134 63.373) (end 62.611 63.373) (width 0.5) (layer "B.Cu") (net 4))
 (segment (start 62.884112 53.955888) (end 62.884112 55.899112) (width 0.5) (layer "B.Cu") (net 4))
 (segment (start 52.11 74.305) (end 52.11 67.397) (width 0.5) (layer "B.Cu") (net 4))
 (segment (start 58.928 77.47) (end 54.61 77.47) (width 0.5) (layer "B.Cu") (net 4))
 (segment (start 61.926371 59.398) (end 61.849 59.398) (width 0.5) (layer "B.Cu") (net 4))
 (segment (start 52.11 74.97) (end 52.11 74.305) (width 0.5) (layer "B.Cu") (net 4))
 (segment (start 61.849 56.934224) (end 62.884112 55.899112) (width 0.5) (layer "B.Cu") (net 4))
 (segment (start 52.11 84.368) (end 52.11 74.305) (width 0.5) (layer "B.Cu") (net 4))
 (segment (start 66.04 50.8) (end 62.884112 53.955888) (width 0.5) (layer "B.Cu") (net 4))
 (segment (start 54.61 77.47) (end 52.11 74.97) (width 0.5) (layer "B.Cu") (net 4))
 (segment (start 55.372 87.63) (end 52.11 84.368) (width 0.5) (layer "B.Cu") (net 4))
 (segment (start 62.611 60.082629) (end 61.926371 59.398) (width 0.5) (layer "B.Cu") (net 4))
 (segment (start 62.611 63.373) (end 62.611 60.082629) (width 0.5) (layer "B.Cu") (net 4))
 (segment (start 59.182 77.216) (end 58.928 77.47) (width 0.5) (layer "B.Cu") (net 4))
 (segment (start 61.253776 54.483) (end 64.262 54.483) (width 0.15) (layer "F.Cu") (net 7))
 (segment (start 60.3 55.91) (end 60.3 55.436776) (width 0.15) (layer "F.Cu") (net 7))
 (segment (start 64.262 54.483) (end 64.389 54.356) (width 0.15) (layer "F.Cu") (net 7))
 (segment (start 60.3 55.436776) (end 61.253776 54.483) (width 0.15) (layer "F.Cu") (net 7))
 (segment (start 59.9 55.91) (end 59.9 55.30402) (width 0.15) (layer "F.Cu") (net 8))
 (segment (start 59.9 55.30402) (end 61.35602 53.848) (width 0.15) (layer "F.Cu") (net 8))
 (segment (start 61.35602 53.848) (end 62.484 53.848) (width 0.15) (layer "F.Cu") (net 8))
 (segment (start 61.089 77.216) (end 62.103 77.216) (width 0.5) (layer "F.Cu") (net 23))
 (segment (start 64.643 84.963) (end 64.897 84.709) (width 0.5) (layer "F.Cu") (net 23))
 (segment (start 62.103 77.216) (end 62.988 77.216) (width 0.5) (layer "F.Cu") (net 23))
 (segment (start 63.308 84.963) (end 64.643 84.963) (width 0.5) (layer "F.Cu") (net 23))
 (via (at 64.897 84.709) (size 0.7) (drill 0.3) (layers "F.Cu" "B.Cu") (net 23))
 (via (at 62.103 77.216) (size 0.7) (drill 0.3) (layers "F.Cu" "B.Cu") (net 23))
 (segment (start 64.897 84.709) (end 64.935371 84.709) (width 0.5) (layer "B.Cu") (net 23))
 (segment (start 62.103 77.216) (end 65.014 74.305) (width 0.5) (layer "B.Cu") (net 23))
 (segment (start 64.935371 84.709) (end 65.753185 83.891186) (width 0.5) (layer "B.Cu") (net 23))
 (segment (start 65.753185 80.866185) (end 62.103 77.216) (width 0.5) (layer "B.Cu") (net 23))
 (segment (start 65.753185 83.891186) (end 65.753185 80.866185) (width 0.5) (layer "B.Cu") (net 23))
 (segment (start 65.014 74.305) (end 67.35 74.305) (width 0.5) (layer "B.Cu") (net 23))
 (segment (start 58.816 55.626) (end 59.1 55.91) (width 0.15) (layer "F.Cu") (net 10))
 (segment (start 57.023 55.626) (end 58.816 55.626) (width 0.15) (layer "F.Cu") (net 10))
 (segment (start 71.724 81.696) (end 71.724 83.089) (width 0.3) (layer "F.Cu") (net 29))
 (segment (start 52.197 70.231) (end 52.197 66.802) (width 0.3) (layer "F.Cu") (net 29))
 (segment (start 65.022 86.233) (end 63.308 86.233) (width 0.3) (layer "F.Cu") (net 29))
 (segment (start 56.003 55.626) (end 56.003 55.622) (width 0.3) (layer "F.Cu") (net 29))
 (segment (start 67.308 83.947) (end 65.784 85.471) (width 0.3) (layer "F.Cu") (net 29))
 (segment (start 65.659 81.788) (end 49.403 81.788) (width 0.3) (layer "F.Cu") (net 29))
 (segment (start 49.403 81.788) (end 49.403 73.025) (width 0.3) (layer "F.Cu") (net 29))
 (segment (start 53.467 65.532) (end 53.467 61.087) (width 0.3) (layer "F.Cu") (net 29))
 (segment (start 65.784 85.471) (end 65.022 86.233) (width 0.3) (layer "F.Cu") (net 29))
 (segment (start 72.394 81.026) (end 71.724 81.696) (width 0.3) (layer "F.Cu") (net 29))
 (segment (start 53.467 61.087) (end 53.34 60.96) (width 0.3) (layer "F.Cu") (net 29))
 (segment (start 52.197 66.802) (end 53.467 65.532) (width 0.3) (layer "F.Cu") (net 29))
 (segment (start 65.784 81.913) (end 65.659 81.788) (width 0.3) (layer "F.Cu") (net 29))
 (segment (start 49.403 73.025) (end 52.197 70.231) (width 0.3) (layer "F.Cu") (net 29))
 (segment (start 70.866 83.947) (end 67.308 83.947) (width 0.3) (layer "F.Cu") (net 29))
 (segment (start 65.784 85.471) (end 65.784 81.913) (width 0.3) (layer "F.Cu") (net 29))
 (segment (start 71.724 83.089) (end 70.866 83.947) (width 0.3) (layer "F.Cu") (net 29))
 (segment (start 56.003 55.622) (end 54.991 54.61) (width 0.3) (layer "F.Cu") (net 29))
 (segment (start 65.669 85.356) (end 65.784 85.471) (width 0.3) (layer "F.Cu") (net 29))
 (via (at 54.991 54.61) (size 0.7) (drill 0.3) (layers "F.Cu" "B.Cu") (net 29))
 (via (at 53.34 60.96) (size 0.7) (drill 0.3) (layers "F.Cu" "B.Cu") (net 29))
 (segment (start 53.34 55.118) (end 53.34 60.96) (width 0.3) (layer "B.Cu") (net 29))
 (segment (start 53.848 54.61) (end 53.34 55.118) (width 0.3) (layer "B.Cu") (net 29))
 (segment (start 54.991 54.61) (end 53.848 54.61) (width 0.3) (layer "B.Cu") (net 29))
 (segment (start 61.929653 61.006348) (end 72.35 71.426695) (width 0.3) (layer "F.Cu") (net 9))
 (segment (start 59.817 53.975) (end 59.5 54.292) (width 0.15) (layer "F.Cu") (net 9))
 (segment (start 61.929652 61.006347) (end 61.595 60.671695) (width 0.3) (layer "F.Cu") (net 9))
 (segment (start 61.595 60.671695) (end 61.595 60.198) (width 0.3) (layer "F.Cu") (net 9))
 (segment (start 72.35 71.426695) (end 72.35 74.305) (width 0.3) (layer "F.Cu") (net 9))
 (segment (start 61.929653 61.006347) (end 61.929653 61.006348) (width 0.3) (layer "F.Cu") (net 9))
 (segment (start 61.929653 61.006347) (end 61.929652 61.006347) (width 0.3) (layer "F.Cu") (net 9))
 (segment (start 59.5 54.292) (end 59.5 55.91) (width 0.15) (layer "F.Cu") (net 9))
 (via (at 61.595 60.198) (size 0.7) (drill 0.3) (layers "F.Cu" "B.Cu") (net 9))
 (via (at 59.817 53.975) (size 0.7) (drill 0.3) (layers "F.Cu" "B.Cu") (free yes) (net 9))
 (segment (start 61.595 60.198) (end 59.817 58.42) (width 0.3) (layer "B.Cu") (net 9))
 (segment (start 59.817 58.42) (end 59.817 53.975) (width 0.3) (layer "B.Cu") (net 9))
 (segment (start 65.784 86.614) (end 64.895 87.503) (width 0.3) (layer "F.Cu") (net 25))
 (segment (start 64.895 87.503) (end 63.308 87.503) (width 0.3) (layer "F.Cu") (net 25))
 (segment (start 67.529 87.284) (end 68.324 86.489) (width 0.3) (layer "F.Cu") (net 25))
 (segment (start 65.784 86.614) (end 66.454 87.284) (width 0.3) (layer "F.Cu") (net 25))
 (segment (start 66.454 87.284) (end 67.529 87.284) (width 0.3) (layer "F.Cu") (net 25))
 (segment (start 63.063 87.491) (end 63.051 87.503) (width 0.3) (layer "F.Cu") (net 25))
 (segment (start 71.37 78.613) (end 71.37 78.359) (width 0.3) (layer "F.Cu") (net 26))
 (segment (start 71.37 75.825) (end 69.85 74.305) (width 0.3) (layer "F.Cu") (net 26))
 (segment (start 71.374 78.363) (end 71.374 81.026) (width 0.3) (layer "F.Cu") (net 26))
 (segment (start 71.37 78.359) (end 71.37 75.825) (width 0.3) (layer "F.Cu") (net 26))
 (segment (start 71.37 78.359) (end 71.374 78.363) (width 0.3) (layer "F.Cu") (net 26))
 (segment (start 66.804 85.471) (end 66.804 86.614) (width 0.3) (layer "F.Cu") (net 24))
 (segment (start 57.023 58.039) (end 57.302 57.76) (width 0.15) (layer "F.Cu") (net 14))
 (segment (start 54.61 62.992) (end 57.023 60.579) (width 0.3) (layer "F.Cu") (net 14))
 (segment (start 54.61 74.305) (end 54.61 62.992) (width 0.3) (layer "F.Cu") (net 14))
 (segment (start 57.302 57.76) (end 58.45 57.76) (width 0.15) (layer "F.Cu") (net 14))
 (via (at 57.023 60.579) (size 0.7) (drill 0.3) (layers "F.Cu" "B.Cu") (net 14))
 (via (at 57.023 58.039) (size 0.7) (drill 0.3) (layers "F.Cu" "B.Cu") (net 14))
 (segment (start 57.023 60.579) (end 57.023 58.039) (width 0.15) (layer "B.Cu") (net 14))
 (segment (start 60.103003 60.325) (end 60.3 60.128003) (width 0.15) (layer "F.Cu") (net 19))
 (segment (start 55.88 58.42) (end 57.785 60.325) (width 0.15) (layer "F.Cu") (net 19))
 (segment (start 57.785 60.325) (end 60.103003 60.325) (width 0.15) (layer "F.Cu") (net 19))
 (segment (start 60.3 60.128003) (end 60.3 58.81) (width 0.15) (layer "F.Cu") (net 19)))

